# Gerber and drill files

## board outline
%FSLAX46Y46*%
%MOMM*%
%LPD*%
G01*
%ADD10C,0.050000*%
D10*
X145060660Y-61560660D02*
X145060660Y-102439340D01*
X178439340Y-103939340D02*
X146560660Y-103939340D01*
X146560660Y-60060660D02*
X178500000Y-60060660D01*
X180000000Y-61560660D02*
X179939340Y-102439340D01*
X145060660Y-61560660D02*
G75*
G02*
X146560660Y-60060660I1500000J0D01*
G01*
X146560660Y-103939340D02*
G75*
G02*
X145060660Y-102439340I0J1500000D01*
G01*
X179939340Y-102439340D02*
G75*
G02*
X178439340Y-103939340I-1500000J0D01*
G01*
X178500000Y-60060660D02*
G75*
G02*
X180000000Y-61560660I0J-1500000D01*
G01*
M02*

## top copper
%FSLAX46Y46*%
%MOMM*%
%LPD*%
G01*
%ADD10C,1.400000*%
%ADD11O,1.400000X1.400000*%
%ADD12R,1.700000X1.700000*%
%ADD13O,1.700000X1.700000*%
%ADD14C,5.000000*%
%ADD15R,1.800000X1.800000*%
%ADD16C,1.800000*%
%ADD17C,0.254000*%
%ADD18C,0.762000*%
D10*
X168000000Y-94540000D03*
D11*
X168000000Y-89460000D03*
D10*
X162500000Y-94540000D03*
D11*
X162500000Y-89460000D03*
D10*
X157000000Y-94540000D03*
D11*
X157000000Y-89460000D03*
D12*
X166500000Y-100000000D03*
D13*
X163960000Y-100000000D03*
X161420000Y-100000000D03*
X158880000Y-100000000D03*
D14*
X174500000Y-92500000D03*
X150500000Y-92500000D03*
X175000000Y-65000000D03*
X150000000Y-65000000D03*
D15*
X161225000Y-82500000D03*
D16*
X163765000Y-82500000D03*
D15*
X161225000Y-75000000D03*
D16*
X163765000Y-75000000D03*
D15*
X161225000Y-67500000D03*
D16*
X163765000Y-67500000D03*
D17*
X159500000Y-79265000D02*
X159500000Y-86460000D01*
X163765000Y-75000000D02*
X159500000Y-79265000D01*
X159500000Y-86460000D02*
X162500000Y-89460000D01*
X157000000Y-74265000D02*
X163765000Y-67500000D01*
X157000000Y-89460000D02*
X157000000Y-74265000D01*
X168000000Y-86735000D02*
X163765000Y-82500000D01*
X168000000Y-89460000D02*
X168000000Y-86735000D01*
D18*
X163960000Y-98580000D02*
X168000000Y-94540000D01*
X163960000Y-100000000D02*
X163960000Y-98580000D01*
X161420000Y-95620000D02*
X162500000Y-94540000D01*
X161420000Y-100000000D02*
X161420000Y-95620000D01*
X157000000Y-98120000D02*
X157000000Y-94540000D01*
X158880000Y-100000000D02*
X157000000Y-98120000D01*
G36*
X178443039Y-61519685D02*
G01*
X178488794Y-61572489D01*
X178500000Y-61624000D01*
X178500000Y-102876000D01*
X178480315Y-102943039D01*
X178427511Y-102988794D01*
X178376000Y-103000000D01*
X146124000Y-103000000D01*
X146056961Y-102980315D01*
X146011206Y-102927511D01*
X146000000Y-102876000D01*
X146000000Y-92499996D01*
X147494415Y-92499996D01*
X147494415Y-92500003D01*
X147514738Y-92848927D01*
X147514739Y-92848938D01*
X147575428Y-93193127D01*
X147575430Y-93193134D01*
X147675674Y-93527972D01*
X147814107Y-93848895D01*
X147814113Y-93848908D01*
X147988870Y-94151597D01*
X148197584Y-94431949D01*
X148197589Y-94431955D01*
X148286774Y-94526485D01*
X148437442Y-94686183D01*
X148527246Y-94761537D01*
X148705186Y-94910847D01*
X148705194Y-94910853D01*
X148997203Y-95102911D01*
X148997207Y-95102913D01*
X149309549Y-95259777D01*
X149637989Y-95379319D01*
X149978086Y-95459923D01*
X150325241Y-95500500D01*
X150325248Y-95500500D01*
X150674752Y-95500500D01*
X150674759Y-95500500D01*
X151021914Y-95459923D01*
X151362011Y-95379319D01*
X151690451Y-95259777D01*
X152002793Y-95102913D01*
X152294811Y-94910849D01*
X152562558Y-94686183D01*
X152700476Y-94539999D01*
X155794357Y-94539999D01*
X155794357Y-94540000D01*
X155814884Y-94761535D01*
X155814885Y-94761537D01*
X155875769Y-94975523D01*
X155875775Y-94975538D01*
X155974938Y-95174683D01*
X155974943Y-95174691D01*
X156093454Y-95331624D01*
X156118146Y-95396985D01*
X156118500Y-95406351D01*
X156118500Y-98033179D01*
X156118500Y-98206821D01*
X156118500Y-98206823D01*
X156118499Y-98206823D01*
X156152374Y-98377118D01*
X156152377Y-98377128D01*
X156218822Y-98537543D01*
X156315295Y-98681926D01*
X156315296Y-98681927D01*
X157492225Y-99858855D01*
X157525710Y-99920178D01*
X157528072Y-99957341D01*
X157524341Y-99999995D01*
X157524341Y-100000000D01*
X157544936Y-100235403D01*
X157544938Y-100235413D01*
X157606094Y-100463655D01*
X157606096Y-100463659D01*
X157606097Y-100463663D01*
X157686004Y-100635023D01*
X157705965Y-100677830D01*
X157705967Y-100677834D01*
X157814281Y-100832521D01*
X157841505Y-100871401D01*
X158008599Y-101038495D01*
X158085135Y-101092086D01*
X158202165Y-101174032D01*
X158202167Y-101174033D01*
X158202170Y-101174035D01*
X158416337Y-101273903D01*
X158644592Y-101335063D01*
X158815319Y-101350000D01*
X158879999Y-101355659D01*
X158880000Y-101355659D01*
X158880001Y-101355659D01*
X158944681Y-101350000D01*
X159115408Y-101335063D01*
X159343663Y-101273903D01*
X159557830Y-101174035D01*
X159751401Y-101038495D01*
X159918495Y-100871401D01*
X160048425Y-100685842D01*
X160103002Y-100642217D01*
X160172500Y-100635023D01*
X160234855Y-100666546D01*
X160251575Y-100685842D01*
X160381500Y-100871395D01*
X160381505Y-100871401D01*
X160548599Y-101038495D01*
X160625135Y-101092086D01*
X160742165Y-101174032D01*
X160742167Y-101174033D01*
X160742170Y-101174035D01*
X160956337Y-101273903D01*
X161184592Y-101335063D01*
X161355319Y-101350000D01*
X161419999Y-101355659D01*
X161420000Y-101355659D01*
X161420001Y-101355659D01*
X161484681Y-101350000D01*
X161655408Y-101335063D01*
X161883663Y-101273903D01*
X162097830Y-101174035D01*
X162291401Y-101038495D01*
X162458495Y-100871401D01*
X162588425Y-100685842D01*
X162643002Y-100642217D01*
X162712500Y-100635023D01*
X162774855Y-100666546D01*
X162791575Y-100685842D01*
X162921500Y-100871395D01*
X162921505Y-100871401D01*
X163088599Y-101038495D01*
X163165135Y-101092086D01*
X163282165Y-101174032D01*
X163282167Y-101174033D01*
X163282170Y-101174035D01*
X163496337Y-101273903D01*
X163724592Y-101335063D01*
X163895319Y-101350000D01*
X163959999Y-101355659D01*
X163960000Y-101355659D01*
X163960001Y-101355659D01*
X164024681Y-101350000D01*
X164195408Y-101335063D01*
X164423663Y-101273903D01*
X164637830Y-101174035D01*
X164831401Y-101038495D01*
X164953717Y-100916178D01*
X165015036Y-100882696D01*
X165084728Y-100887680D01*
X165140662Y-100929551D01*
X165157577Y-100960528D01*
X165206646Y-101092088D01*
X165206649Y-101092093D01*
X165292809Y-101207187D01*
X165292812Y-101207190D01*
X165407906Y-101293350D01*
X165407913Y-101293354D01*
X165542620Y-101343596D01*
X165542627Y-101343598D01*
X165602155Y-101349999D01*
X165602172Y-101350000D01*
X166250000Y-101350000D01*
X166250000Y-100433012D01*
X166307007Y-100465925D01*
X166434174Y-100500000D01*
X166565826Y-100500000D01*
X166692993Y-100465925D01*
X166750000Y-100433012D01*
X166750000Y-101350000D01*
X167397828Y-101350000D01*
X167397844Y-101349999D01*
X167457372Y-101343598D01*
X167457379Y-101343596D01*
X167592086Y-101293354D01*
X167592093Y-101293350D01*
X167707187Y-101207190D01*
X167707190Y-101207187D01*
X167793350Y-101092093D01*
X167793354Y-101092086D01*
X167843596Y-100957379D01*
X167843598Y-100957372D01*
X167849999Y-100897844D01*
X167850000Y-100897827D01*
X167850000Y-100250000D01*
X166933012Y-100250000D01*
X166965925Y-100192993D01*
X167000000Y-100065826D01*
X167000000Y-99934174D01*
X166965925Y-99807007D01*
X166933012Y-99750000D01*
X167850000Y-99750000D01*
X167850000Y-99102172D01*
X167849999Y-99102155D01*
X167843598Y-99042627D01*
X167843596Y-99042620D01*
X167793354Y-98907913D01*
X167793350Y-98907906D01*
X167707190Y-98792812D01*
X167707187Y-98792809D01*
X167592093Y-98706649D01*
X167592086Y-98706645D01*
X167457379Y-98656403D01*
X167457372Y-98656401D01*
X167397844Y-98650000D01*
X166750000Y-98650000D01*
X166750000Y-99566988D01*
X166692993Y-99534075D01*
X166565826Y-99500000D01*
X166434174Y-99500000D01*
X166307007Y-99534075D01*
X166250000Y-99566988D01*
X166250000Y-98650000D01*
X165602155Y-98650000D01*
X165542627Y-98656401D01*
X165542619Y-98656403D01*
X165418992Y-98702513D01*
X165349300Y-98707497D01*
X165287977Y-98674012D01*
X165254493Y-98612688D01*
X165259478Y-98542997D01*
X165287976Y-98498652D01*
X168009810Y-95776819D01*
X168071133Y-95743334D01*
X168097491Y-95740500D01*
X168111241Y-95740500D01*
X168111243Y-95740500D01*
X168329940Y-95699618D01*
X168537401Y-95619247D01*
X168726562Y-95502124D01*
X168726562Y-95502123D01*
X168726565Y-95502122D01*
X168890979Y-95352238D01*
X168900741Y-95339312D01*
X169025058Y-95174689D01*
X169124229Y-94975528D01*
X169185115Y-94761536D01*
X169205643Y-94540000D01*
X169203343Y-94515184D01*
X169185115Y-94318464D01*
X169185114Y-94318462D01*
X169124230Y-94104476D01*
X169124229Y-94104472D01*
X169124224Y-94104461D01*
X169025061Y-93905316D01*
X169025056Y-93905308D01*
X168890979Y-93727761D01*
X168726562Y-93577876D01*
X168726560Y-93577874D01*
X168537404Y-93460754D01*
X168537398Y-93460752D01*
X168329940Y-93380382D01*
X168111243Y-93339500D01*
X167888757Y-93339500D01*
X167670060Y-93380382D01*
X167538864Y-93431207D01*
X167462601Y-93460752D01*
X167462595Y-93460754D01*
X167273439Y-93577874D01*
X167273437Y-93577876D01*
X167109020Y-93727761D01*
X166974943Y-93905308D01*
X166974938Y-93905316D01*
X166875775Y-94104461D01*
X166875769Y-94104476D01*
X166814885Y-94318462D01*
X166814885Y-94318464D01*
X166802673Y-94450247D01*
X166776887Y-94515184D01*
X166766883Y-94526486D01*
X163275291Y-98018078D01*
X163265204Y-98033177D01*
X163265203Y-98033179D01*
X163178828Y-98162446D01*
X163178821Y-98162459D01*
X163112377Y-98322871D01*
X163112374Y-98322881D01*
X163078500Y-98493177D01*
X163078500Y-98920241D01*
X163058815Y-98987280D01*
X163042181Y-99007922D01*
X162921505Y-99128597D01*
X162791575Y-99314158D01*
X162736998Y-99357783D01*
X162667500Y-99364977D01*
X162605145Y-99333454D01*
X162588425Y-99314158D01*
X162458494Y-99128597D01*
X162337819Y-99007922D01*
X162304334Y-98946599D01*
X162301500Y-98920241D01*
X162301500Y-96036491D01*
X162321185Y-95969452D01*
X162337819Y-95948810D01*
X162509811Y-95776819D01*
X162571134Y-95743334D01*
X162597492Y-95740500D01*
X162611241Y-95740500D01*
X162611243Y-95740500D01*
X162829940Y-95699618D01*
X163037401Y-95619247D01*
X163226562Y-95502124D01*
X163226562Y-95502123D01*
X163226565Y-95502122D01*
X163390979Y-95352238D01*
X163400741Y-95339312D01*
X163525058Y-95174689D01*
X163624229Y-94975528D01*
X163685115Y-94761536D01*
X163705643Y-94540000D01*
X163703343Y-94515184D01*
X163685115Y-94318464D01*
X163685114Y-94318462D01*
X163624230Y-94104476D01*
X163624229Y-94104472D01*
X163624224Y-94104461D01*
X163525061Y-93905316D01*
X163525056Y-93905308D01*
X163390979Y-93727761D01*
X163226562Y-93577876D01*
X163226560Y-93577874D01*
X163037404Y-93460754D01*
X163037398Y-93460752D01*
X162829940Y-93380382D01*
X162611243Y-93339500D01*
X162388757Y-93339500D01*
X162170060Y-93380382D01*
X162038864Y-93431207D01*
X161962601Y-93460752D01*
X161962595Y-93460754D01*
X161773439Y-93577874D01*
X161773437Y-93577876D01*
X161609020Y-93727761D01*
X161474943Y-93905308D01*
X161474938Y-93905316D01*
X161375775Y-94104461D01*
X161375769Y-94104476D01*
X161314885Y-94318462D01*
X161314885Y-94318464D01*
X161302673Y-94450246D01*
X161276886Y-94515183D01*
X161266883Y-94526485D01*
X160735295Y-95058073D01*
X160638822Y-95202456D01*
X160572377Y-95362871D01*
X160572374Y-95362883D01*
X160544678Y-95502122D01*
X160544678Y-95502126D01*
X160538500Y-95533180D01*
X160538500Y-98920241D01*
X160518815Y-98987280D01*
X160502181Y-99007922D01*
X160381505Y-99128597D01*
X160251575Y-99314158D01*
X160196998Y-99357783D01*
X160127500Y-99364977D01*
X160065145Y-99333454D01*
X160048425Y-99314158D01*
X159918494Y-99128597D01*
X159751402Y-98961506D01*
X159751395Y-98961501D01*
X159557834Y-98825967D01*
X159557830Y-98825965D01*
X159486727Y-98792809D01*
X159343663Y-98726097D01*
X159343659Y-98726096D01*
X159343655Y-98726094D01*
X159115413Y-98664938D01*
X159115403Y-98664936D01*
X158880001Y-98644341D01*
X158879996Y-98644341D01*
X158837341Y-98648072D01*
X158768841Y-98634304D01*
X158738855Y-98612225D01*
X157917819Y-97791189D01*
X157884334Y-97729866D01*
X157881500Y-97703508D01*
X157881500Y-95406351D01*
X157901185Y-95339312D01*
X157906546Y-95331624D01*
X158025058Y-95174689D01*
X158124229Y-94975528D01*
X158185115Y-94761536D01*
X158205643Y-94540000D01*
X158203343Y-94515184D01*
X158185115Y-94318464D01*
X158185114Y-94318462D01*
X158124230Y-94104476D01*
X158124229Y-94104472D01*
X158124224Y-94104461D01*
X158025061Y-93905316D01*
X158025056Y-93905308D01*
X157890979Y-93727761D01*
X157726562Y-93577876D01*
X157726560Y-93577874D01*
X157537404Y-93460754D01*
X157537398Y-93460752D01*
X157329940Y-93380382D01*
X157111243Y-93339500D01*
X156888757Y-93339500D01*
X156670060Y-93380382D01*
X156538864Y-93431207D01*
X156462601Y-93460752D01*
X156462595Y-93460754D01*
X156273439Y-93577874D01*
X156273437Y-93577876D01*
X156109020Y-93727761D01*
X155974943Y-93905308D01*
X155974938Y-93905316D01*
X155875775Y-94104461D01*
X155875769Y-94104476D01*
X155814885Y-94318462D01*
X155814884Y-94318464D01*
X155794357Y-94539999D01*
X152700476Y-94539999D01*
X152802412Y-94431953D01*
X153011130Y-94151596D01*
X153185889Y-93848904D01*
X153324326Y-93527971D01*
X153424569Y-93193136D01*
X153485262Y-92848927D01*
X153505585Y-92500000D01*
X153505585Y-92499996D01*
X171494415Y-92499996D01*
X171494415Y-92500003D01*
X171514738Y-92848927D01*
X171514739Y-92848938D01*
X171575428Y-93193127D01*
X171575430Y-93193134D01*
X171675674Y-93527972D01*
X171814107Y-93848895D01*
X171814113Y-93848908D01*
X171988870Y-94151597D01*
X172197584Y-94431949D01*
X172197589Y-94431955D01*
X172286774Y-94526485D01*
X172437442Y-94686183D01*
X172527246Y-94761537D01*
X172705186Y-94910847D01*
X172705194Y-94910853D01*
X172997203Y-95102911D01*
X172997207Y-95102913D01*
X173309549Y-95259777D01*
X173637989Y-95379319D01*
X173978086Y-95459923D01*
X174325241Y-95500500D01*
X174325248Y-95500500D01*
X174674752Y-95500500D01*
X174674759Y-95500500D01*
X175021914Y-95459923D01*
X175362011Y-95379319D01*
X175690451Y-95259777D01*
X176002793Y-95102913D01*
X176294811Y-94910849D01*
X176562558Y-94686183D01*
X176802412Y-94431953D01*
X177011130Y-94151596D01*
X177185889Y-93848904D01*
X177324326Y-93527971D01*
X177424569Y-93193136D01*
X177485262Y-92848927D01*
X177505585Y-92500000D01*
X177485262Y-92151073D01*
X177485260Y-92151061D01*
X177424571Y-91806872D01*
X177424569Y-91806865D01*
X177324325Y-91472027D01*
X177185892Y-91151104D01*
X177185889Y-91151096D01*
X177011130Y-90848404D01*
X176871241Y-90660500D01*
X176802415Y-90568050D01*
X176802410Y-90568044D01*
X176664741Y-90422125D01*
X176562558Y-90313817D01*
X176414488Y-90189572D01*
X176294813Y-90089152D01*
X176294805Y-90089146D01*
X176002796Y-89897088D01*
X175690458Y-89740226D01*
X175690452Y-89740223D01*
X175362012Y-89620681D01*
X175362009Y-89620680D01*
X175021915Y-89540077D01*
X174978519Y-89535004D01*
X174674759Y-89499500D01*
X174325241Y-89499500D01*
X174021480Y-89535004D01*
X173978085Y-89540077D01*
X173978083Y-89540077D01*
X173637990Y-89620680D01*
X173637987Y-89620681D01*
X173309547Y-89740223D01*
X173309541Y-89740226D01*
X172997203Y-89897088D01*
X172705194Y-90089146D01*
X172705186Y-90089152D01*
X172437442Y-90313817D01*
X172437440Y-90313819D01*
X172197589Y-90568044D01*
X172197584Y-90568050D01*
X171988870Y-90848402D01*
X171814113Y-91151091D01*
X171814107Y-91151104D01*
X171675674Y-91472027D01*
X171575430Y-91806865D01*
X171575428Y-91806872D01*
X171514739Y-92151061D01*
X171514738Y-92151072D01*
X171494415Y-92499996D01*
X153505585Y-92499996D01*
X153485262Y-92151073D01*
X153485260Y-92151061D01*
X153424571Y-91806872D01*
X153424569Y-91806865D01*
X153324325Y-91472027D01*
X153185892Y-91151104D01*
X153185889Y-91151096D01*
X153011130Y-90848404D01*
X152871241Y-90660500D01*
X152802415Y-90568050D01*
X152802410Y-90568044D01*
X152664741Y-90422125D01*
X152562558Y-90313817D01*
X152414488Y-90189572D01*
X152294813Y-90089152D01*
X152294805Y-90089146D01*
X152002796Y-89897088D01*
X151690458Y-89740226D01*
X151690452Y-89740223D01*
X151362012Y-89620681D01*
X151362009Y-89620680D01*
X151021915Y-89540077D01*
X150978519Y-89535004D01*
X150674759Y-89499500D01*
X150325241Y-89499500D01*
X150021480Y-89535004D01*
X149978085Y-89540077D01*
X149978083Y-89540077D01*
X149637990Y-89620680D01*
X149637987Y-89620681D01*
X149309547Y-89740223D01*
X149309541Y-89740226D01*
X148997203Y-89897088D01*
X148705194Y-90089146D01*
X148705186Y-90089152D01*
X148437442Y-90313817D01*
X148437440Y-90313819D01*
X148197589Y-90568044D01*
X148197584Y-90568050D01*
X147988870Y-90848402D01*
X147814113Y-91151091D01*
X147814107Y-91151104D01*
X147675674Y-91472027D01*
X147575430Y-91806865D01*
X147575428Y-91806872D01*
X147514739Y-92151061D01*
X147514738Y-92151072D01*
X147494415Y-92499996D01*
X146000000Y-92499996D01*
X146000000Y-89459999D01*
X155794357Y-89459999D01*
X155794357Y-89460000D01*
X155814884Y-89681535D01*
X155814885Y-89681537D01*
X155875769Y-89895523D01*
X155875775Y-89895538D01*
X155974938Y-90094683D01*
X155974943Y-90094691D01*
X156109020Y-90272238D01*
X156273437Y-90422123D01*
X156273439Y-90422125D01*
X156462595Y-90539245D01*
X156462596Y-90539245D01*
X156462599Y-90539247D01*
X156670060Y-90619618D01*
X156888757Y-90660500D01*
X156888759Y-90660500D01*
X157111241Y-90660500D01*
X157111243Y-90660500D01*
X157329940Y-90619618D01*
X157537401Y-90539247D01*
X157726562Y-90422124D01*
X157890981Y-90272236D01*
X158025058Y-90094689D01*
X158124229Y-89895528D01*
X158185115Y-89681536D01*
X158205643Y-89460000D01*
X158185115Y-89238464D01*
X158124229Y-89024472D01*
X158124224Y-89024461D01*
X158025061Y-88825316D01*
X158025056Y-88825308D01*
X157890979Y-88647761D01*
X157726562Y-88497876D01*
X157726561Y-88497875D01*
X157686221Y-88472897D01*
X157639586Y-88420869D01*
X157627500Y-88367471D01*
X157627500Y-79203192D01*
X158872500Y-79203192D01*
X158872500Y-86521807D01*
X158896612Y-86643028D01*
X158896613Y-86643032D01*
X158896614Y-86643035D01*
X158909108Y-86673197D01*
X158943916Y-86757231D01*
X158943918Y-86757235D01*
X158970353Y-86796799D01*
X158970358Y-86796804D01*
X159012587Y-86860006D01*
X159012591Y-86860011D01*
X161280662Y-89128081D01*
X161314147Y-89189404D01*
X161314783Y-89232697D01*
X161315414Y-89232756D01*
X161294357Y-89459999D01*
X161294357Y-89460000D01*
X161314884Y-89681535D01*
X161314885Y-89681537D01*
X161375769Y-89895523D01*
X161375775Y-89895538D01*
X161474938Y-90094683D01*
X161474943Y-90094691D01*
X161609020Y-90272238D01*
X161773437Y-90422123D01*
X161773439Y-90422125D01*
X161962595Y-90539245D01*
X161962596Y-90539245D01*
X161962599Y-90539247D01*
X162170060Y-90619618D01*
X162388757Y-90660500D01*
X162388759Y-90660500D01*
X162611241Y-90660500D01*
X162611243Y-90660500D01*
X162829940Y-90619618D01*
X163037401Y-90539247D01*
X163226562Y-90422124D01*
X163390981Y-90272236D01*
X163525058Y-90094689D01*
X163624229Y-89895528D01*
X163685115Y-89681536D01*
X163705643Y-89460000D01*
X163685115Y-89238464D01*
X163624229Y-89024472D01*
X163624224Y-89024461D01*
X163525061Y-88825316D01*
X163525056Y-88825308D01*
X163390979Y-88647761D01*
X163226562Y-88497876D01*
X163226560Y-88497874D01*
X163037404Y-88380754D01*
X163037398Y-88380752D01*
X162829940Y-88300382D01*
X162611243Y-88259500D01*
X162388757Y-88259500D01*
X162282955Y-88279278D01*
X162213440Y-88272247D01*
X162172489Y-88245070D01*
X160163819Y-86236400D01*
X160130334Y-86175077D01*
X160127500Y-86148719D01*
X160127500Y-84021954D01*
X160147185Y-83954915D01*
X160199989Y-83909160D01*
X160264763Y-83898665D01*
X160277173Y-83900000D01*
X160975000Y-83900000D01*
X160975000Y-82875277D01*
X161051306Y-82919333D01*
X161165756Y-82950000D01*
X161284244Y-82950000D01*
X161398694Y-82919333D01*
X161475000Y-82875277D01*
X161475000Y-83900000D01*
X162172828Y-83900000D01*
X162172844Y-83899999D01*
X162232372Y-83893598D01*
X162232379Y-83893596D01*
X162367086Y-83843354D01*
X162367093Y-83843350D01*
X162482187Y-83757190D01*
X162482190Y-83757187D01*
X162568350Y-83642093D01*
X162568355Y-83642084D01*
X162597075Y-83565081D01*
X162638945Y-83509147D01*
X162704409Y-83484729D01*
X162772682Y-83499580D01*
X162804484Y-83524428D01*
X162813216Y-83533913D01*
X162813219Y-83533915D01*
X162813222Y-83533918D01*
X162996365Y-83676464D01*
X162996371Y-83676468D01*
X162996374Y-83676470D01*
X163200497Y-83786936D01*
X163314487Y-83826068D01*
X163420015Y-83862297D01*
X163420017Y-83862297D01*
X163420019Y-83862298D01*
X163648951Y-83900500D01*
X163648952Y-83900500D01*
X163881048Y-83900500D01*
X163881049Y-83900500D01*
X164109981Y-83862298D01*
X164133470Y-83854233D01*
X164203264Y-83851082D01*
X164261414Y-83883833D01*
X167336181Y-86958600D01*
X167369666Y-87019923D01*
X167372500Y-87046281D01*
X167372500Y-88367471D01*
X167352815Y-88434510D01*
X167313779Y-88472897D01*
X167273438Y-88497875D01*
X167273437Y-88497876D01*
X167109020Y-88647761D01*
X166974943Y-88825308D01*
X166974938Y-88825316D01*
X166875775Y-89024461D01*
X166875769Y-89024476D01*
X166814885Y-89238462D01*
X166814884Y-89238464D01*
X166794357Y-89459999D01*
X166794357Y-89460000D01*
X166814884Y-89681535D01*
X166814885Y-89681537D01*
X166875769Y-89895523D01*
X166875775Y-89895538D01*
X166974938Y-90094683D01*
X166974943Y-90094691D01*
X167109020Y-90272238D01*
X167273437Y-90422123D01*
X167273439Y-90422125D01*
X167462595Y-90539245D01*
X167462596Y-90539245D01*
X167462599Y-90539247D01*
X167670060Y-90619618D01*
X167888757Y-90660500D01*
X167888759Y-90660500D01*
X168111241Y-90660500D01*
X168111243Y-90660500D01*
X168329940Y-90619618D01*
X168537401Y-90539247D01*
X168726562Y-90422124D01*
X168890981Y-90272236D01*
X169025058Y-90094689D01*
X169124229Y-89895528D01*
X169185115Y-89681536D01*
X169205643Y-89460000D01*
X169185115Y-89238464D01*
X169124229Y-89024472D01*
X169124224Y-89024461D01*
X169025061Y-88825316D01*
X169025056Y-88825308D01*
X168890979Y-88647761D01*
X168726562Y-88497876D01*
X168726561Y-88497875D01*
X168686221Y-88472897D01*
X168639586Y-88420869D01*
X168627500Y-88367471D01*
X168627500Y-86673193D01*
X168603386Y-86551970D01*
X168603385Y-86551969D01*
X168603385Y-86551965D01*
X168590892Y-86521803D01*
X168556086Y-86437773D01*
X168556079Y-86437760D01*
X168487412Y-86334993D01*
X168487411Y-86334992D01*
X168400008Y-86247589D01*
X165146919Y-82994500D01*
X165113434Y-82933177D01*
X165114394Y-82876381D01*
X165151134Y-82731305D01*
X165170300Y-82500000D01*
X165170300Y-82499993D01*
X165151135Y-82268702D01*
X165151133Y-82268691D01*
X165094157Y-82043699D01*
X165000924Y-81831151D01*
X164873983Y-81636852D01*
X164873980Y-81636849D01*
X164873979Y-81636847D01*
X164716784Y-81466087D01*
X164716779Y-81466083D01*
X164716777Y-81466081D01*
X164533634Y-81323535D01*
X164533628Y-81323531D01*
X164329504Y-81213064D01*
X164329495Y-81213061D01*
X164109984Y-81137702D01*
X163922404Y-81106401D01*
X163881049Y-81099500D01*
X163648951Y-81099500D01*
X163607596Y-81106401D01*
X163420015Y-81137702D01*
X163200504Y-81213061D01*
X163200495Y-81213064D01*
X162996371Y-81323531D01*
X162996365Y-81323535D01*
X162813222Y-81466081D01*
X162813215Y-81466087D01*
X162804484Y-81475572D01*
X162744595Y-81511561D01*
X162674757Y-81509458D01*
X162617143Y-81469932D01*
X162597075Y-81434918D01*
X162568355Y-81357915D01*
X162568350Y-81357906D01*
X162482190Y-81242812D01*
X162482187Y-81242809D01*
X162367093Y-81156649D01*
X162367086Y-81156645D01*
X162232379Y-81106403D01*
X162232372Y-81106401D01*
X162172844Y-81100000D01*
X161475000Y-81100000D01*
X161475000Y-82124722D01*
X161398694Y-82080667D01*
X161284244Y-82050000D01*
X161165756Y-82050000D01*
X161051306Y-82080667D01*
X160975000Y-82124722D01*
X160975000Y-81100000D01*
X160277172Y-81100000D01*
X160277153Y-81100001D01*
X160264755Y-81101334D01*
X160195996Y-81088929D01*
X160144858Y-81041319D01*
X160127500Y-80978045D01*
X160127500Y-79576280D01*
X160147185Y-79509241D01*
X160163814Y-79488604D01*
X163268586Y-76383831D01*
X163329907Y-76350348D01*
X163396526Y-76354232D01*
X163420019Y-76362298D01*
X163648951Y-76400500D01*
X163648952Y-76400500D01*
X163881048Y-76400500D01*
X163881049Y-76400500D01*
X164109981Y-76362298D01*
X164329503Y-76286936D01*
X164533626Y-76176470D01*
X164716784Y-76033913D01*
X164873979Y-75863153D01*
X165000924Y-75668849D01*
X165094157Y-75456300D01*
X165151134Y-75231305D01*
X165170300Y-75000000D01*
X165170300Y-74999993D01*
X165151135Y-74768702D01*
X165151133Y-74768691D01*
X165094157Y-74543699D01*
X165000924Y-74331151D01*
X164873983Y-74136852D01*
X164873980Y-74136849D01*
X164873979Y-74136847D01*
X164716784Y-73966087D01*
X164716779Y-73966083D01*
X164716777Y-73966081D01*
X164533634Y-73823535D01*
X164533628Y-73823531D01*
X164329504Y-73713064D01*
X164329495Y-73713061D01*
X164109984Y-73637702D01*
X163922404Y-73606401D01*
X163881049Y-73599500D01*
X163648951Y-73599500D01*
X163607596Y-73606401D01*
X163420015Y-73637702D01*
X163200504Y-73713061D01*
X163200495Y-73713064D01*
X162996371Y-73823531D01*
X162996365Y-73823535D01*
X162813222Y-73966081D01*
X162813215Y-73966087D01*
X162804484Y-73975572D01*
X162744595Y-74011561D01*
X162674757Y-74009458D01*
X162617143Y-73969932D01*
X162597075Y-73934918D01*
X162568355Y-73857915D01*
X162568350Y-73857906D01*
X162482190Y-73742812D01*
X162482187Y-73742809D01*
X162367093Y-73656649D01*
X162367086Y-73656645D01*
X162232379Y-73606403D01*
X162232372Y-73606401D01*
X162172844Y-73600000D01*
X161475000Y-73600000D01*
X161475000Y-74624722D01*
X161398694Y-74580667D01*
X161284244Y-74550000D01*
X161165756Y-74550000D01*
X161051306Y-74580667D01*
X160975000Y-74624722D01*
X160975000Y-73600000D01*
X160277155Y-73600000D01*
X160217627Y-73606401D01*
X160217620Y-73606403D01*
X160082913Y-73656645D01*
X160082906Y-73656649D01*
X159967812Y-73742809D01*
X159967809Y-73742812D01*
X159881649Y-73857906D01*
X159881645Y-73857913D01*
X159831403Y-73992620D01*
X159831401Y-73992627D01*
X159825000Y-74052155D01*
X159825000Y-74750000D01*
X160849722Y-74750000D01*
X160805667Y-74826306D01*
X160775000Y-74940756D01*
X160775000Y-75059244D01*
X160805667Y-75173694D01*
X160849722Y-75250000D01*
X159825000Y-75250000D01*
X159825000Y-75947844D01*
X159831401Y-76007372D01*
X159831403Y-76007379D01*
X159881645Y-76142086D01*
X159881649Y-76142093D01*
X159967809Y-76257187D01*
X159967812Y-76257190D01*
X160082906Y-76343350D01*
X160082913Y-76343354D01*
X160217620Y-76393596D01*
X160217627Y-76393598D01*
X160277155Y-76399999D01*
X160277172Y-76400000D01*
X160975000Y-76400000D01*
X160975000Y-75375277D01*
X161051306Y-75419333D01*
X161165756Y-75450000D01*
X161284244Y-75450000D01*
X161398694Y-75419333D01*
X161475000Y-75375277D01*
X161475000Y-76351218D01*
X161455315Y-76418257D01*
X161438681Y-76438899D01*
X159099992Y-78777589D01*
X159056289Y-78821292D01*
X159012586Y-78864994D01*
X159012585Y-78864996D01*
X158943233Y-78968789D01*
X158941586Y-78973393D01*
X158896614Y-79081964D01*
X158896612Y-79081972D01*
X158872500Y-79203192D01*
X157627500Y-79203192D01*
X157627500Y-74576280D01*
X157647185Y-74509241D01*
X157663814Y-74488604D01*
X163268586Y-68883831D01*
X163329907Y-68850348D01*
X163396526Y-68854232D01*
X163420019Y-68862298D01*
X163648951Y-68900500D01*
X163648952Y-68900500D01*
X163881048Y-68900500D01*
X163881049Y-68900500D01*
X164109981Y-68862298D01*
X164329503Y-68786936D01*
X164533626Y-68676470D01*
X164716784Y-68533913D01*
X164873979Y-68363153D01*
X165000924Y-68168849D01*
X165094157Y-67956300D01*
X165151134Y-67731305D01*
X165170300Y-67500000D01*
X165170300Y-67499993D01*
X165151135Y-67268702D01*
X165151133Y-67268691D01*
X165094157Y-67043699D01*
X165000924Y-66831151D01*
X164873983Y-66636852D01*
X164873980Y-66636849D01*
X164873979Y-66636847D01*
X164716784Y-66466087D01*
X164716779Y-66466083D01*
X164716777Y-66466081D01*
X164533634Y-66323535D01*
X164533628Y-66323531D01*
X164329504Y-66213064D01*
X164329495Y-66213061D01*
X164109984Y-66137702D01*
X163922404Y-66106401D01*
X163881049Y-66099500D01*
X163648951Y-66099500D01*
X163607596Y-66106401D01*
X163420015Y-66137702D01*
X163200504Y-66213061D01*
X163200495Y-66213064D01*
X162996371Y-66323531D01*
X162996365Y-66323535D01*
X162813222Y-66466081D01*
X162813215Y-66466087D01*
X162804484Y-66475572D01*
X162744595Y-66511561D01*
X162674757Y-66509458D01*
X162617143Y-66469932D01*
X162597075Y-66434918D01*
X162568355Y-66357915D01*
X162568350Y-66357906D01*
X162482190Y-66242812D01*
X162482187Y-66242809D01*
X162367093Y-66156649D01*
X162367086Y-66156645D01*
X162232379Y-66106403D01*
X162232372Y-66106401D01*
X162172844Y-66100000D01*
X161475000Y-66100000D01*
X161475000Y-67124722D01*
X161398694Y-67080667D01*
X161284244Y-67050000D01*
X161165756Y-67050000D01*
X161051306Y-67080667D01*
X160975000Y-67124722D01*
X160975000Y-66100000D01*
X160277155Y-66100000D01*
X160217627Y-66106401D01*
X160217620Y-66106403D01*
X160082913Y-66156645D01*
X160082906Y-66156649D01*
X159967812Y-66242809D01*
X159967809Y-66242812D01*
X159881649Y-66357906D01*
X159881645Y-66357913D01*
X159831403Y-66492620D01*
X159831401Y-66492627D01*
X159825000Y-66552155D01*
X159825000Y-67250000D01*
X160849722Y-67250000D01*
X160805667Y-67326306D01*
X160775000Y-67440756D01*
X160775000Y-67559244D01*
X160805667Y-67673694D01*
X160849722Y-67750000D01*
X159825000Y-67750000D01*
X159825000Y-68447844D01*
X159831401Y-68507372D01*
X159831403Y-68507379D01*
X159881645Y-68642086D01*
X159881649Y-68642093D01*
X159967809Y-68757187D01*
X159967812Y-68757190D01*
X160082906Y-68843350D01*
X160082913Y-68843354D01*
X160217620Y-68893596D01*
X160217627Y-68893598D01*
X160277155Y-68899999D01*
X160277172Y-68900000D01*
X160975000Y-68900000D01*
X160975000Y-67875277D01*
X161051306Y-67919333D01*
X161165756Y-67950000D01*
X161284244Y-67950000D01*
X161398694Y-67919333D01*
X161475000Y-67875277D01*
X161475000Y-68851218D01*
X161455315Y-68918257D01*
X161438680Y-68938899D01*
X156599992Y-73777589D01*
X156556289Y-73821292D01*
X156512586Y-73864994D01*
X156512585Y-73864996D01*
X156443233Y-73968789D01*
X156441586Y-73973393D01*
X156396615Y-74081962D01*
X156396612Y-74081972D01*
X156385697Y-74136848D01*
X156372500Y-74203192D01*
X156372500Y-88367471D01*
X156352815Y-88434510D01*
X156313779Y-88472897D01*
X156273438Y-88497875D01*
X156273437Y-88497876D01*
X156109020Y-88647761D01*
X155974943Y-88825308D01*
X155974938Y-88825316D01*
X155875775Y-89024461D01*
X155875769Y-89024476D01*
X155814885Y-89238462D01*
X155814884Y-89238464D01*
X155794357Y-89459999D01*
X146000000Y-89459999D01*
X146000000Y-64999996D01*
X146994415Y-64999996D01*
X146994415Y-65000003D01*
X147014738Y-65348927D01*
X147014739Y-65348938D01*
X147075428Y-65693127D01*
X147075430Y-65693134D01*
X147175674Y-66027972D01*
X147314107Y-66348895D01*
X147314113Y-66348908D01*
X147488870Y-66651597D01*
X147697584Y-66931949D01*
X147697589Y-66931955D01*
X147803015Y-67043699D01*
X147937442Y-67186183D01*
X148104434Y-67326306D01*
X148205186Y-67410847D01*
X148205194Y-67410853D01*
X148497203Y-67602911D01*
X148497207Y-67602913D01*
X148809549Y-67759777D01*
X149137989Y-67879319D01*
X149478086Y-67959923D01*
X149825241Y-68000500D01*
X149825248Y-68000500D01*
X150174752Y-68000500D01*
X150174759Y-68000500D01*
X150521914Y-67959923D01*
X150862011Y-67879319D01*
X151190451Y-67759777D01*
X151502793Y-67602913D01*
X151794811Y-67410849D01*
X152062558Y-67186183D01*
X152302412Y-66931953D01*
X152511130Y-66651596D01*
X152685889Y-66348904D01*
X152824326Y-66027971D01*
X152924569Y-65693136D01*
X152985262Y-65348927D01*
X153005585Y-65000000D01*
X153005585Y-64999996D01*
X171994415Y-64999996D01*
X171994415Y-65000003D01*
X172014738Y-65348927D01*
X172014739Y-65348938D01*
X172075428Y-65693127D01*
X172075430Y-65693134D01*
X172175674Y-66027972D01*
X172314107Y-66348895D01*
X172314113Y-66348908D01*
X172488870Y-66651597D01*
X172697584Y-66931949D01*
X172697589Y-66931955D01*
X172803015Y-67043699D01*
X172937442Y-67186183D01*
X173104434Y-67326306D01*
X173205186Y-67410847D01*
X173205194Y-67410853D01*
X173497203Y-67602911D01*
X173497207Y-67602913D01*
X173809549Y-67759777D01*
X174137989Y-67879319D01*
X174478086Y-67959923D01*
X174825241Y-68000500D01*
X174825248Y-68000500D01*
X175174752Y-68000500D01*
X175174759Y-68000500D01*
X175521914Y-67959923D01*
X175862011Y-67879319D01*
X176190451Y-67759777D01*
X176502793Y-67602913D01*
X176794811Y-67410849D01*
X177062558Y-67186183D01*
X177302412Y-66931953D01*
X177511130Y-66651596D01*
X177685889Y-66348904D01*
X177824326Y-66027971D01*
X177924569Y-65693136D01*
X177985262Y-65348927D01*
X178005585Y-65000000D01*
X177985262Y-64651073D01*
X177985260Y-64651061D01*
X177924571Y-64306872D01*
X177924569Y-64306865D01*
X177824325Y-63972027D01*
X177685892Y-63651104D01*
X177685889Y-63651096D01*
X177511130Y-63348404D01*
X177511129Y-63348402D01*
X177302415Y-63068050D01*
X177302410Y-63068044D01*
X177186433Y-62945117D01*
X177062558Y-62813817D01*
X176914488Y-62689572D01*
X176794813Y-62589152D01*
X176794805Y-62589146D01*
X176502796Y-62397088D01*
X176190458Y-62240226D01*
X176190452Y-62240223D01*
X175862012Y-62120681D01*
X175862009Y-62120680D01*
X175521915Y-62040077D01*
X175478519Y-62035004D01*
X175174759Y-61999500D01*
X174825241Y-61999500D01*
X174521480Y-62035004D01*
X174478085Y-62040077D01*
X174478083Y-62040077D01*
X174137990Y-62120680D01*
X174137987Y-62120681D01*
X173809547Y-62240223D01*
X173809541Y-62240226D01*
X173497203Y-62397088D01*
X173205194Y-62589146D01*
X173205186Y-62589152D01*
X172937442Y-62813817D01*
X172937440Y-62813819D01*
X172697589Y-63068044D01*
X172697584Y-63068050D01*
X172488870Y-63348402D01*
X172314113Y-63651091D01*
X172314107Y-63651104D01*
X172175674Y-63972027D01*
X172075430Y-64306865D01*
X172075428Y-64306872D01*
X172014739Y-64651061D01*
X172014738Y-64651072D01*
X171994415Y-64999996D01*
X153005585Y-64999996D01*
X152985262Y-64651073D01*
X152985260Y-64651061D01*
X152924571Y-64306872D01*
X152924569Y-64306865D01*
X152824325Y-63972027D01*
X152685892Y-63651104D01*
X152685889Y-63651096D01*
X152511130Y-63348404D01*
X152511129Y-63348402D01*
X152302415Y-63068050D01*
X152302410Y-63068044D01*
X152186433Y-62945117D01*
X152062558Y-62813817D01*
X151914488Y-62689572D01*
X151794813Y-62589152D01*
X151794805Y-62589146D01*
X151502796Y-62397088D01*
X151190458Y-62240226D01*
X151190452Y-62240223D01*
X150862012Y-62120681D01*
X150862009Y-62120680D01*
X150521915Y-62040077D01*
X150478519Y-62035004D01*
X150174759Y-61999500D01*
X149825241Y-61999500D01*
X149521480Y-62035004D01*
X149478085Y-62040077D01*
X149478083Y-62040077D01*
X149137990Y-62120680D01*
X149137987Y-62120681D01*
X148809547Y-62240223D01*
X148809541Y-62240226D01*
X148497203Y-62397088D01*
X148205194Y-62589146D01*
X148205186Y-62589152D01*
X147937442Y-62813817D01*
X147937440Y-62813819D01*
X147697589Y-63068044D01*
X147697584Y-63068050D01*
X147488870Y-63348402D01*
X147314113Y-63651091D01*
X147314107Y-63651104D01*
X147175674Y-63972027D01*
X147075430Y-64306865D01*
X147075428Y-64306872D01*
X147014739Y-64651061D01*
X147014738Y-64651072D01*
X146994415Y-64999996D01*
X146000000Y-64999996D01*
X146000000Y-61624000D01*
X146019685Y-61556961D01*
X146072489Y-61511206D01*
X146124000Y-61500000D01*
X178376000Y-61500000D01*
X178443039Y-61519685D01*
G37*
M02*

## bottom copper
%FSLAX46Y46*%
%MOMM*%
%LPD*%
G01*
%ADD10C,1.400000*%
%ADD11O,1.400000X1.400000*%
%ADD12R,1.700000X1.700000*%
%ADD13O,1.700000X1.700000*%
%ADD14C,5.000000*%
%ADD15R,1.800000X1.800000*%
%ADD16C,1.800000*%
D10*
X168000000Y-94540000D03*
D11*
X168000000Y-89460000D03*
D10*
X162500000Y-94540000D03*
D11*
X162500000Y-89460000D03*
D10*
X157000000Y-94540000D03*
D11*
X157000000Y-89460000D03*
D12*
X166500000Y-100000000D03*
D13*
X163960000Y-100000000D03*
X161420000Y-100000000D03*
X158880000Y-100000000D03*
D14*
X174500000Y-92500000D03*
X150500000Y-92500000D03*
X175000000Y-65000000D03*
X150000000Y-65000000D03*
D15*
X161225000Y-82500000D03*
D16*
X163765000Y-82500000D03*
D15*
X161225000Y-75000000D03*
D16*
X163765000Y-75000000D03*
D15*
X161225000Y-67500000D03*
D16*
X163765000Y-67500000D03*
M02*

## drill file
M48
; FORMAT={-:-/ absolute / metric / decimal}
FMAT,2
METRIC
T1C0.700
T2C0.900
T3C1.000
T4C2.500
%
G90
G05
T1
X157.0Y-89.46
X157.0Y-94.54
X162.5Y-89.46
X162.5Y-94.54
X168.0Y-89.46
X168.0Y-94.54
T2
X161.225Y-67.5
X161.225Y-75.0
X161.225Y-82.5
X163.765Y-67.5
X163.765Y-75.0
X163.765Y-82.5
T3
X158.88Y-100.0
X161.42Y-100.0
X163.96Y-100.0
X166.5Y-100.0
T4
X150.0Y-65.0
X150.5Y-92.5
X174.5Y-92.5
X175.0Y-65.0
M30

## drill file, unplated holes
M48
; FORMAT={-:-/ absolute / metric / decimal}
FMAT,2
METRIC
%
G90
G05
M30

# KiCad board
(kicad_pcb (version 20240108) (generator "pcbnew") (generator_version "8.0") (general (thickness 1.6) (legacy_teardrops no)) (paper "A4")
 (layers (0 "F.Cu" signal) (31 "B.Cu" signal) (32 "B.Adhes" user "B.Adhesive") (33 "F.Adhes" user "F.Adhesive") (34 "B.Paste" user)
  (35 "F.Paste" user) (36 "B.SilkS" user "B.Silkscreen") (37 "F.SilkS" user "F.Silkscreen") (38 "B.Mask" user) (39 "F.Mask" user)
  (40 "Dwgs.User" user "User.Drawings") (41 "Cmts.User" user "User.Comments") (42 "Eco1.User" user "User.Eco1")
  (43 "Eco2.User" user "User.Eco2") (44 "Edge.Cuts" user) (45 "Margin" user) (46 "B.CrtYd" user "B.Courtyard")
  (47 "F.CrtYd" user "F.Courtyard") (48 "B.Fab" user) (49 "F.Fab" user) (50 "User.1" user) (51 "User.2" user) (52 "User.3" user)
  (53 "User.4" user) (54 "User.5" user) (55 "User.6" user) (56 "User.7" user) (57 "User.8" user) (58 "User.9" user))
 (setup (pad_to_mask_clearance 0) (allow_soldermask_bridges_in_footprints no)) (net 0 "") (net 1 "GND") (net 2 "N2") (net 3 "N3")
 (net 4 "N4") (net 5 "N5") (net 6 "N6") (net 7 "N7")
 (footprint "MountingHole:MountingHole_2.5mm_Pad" (layer "F.Cu") (at 175 65)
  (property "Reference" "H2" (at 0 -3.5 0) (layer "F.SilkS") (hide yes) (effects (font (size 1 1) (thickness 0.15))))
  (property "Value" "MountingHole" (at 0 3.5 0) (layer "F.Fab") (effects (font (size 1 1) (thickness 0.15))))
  (pad "1" thru_hole circle (at 0 0) (size 5 5) (drill 2.5) (layers "*.Cu" "*.Mask") (remove_unused_layers no)))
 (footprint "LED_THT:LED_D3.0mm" (layer "F.Cu") (at 161.225 67.5)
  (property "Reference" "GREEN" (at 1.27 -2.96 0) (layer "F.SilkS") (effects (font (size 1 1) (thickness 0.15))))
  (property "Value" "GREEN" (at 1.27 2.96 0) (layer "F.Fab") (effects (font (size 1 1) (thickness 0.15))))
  (pad "1" thru_hole rect (at 0 0) (size 1.8 1.8) (drill 0.9) (layers "*.Cu" "*.Mask") (remove_unused_layers no) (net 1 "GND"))
  (pad "2" thru_hole circle (at 2.54 0) (size 1.8 1.8) (drill 0.9) (layers "*.Cu" "*.Mask") (remove_unused_layers no) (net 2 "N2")))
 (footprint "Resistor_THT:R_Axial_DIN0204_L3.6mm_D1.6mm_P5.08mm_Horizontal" (layer "F.Cu") (at 168 94.54 90)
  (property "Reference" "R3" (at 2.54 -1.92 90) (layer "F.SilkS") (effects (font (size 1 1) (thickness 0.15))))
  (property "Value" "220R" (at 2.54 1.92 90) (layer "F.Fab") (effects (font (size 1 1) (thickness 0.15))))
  (pad "1" thru_hole circle (at 0 0 90) (size 1.4 1.4) (drill 0.7) (layers "*.Cu" "*.Mask") (remove_unused_layers no) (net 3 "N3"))
  (pad "2" thru_hole oval (at 5.08 0 90) (size 1.4 1.4) (drill 0.7) (layers "*.Cu" "*.Mask") (remove_unused_layers no) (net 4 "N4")))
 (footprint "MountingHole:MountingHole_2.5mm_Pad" (layer "F.Cu") (at 150 65)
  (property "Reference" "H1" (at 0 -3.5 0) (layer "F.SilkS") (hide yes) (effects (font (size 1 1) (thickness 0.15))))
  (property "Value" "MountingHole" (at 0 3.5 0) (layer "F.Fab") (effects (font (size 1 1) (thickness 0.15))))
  (pad "1" thru_hole circle (at 0 0) (size 5 5) (drill 2.5) (layers "*.Cu" "*.Mask") (remove_unused_layers no)))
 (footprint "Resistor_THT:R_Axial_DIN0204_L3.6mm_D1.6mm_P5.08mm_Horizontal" (layer "F.Cu") (at 162.5 94.54 90)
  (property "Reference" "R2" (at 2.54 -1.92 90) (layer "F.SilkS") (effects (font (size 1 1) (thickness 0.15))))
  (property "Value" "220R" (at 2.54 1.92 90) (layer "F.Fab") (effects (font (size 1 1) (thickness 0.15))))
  (pad "1" thru_hole circle (at 0 0 90) (size 1.4 1.4) (drill 0.7) (layers "*.Cu" "*.Mask") (remove_unused_layers no) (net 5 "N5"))
  (pad "2" thru_hole oval (at 5.08 0 90) (size 1.4 1.4) (drill 0.7) (layers "*.Cu" "*.Mask") (remove_unused_layers no) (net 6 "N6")))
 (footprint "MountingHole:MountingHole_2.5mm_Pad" (layer "F.Cu") (at 150.5 92.5)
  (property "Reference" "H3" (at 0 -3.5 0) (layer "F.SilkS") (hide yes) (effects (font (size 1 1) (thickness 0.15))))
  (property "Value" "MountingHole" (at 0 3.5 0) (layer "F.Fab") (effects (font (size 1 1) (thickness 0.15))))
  (pad "1" thru_hole circle (at 0 0) (size 5 5) (drill 2.5) (layers "*.Cu" "*.Mask") (remove_unused_layers no)))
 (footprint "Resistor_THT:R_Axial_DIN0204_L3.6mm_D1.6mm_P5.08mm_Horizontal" (layer "F.Cu") (at 157 94.54 90)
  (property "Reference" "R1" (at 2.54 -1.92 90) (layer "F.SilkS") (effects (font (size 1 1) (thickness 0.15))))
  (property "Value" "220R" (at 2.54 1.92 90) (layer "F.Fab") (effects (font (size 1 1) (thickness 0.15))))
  (pad "1" thru_hole circle (at 0 0 90) (size 1.4 1.4) (drill 0.7) (layers "*.Cu" "*.Mask") (remove_unused_layers no) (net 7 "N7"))
  (pad "2" thru_hole oval (at 5.08 0 90) (size 1.4 1.4) (drill 0.7) (layers "*.Cu" "*.Mask") (remove_unused_layers no) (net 2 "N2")))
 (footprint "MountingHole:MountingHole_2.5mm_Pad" (layer "F.Cu") (at 174.5 92.5)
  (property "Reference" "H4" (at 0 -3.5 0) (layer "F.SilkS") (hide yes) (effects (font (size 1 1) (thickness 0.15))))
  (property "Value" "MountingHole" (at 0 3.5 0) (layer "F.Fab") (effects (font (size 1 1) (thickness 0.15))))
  (pad "1" thru_hole circle (at 0 0) (size 5 5) (drill 2.5) (layers "*.Cu" "*.Mask") (remove_unused_layers no)))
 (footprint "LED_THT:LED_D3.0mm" (layer "F.Cu") (at 161.225 82.5)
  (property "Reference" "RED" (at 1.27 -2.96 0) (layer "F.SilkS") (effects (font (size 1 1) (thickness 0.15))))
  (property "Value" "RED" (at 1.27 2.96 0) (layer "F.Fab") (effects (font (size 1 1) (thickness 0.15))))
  (pad "1" thru_hole rect (at 0 0) (size 1.8 1.8) (drill 0.9) (layers "*.Cu" "*.Mask") (remove_unused_layers no) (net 1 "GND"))
  (pad "2" thru_hole circle (at 2.54 0) (size 1.8 1.8) (drill 0.9) (layers "*.Cu" "*.Mask") (remove_unused_layers no) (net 4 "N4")))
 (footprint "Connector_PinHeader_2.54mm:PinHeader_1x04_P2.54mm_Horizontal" (layer "F.Cu") (at 166.5 100 -90)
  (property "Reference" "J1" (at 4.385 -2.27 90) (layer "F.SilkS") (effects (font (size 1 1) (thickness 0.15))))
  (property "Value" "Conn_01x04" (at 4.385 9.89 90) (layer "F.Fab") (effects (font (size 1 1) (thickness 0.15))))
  (pad "1" thru_hole rect (at 0 0 270) (size 1.7 1.7) (drill 1) (layers "*.Cu" "*.Mask") (remove_unused_layers no) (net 1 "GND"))
  (pad "2" thru_hole oval (at 0 2.54 270) (size 1.7 1.7) (drill 1) (layers "*.Cu" "*.Mask") (remove_unused_layers no) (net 3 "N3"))
  (pad "3" thru_hole oval (at 0 5.08 270) (size 1.7 1.7) (drill 1) (layers "*.Cu" "*.Mask") (remove_unused_layers no) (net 5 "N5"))
  (pad "4" thru_hole oval (at 0 7.62 270) (size 1.7 1.7) (drill 1) (layers "*.Cu" "*.Mask") (remove_unused_layers no) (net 7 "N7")))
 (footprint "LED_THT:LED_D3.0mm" (layer "F.Cu") (at 161.225 75)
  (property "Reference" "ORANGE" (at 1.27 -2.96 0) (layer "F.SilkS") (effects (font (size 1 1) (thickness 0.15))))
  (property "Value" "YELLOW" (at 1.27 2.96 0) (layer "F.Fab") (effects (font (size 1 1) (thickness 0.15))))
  (pad "1" thru_hole rect (at 0 0) (size 1.8 1.8) (drill 0.9) (layers "*.Cu" "*.Mask") (remove_unused_layers no) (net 1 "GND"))
  (pad "2" thru_hole circle (at 2.54 0) (size 1.8 1.8) (drill 0.9) (layers "*.Cu" "*.Mask") (remove_unused_layers no) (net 6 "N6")))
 (gr_arc (start 145.06066 61.56066) (mid 145.5 60.5) (end 146.56066 60.06066) (stroke (width 0.05) (type default)) (layer "Edge.Cuts"))
 (gr_line (start 145.06066 61.56066) (end 145.06066 102.43934) (stroke (width 0.05) (type default)) (layer "Edge.Cuts"))
 (gr_arc (start 179.93934 102.43934) (mid 179.5 103.5) (end 178.43934 103.93934) (stroke (width 0.05) (type default)) (layer "Edge.Cuts"))
 (gr_line (start 180 61.56066) (end 179.93934 102.43934) (stroke (width 0.05) (type default)) (layer "Edge.Cuts"))
 (gr_arc (start 146.56066 103.93934) (mid 145.5 103.5) (end 145.06066 102.43934) (stroke (width 0.05) (type default)) (layer "Edge.Cuts"))
 (gr_arc (start 178.5 60.06066) (mid 179.56066 60.5) (end 180 61.56066) (stroke (width 0.05) (type default)) (layer "Edge.Cuts"))
 (gr_line (start 146.56066 60.06066) (end 178.5 60.06066) (stroke (width 0.05) (type default)) (layer "Edge.Cuts"))
 (gr_line (start 178.43934 103.93934) (end 146.56066 103.93934) (stroke (width 0.05) (type default)) (layer "Edge.Cuts"))
 (segment (start 157 74.265) (end 163.765 67.5) (width 0.254) (layer "F.Cu") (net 2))
 (segment (start 157 89.46) (end 157 74.265) (width 0.254) (layer "F.Cu") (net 2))
 (segment (start 159.5 79.265) (end 159.5 86.46) (width 0.254) (layer "F.Cu") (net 6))
 (segment (start 163.765 75) (end 159.5 79.265) (width 0.254) (layer "F.Cu") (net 6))
 (segment (start 159.5 86.46) (end 162.5 89.46) (width 0.254) (layer "F.Cu") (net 6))
 (segment (start 168 86.735) (end 163.765 82.5) (width 0.254) (layer "F.Cu") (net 4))
 (segment (start 168 89.46) (end 168 86.735) (width 0.254) (layer "F.Cu") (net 4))
 (segment (start 161.42 100) (end 161.42 95.62) (width 0.762) (layer "F.Cu") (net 5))
 (segment (start 161.42 95.62) (end 162.5 94.54) (width 0.762) (layer "F.Cu") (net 5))
 (segment (start 158.88 100) (end 157 98.12) (width 0.762) (layer "F.Cu") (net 7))
 (segment (start 157 98.12) (end 157 94.54) (width 0.762) (layer "F.Cu") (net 7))
 (segment (start 163.96 98.58) (end 168 94.54) (width 0.762) (layer "F.Cu") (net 3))
 (segment (start 163.96 100) (end 163.96 98.58) (width 0.762) (layer "F.Cu") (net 3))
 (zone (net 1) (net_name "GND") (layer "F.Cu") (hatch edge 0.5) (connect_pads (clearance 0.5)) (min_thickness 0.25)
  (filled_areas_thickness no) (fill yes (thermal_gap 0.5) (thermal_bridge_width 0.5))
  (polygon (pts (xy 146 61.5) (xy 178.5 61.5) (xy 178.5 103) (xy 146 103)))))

